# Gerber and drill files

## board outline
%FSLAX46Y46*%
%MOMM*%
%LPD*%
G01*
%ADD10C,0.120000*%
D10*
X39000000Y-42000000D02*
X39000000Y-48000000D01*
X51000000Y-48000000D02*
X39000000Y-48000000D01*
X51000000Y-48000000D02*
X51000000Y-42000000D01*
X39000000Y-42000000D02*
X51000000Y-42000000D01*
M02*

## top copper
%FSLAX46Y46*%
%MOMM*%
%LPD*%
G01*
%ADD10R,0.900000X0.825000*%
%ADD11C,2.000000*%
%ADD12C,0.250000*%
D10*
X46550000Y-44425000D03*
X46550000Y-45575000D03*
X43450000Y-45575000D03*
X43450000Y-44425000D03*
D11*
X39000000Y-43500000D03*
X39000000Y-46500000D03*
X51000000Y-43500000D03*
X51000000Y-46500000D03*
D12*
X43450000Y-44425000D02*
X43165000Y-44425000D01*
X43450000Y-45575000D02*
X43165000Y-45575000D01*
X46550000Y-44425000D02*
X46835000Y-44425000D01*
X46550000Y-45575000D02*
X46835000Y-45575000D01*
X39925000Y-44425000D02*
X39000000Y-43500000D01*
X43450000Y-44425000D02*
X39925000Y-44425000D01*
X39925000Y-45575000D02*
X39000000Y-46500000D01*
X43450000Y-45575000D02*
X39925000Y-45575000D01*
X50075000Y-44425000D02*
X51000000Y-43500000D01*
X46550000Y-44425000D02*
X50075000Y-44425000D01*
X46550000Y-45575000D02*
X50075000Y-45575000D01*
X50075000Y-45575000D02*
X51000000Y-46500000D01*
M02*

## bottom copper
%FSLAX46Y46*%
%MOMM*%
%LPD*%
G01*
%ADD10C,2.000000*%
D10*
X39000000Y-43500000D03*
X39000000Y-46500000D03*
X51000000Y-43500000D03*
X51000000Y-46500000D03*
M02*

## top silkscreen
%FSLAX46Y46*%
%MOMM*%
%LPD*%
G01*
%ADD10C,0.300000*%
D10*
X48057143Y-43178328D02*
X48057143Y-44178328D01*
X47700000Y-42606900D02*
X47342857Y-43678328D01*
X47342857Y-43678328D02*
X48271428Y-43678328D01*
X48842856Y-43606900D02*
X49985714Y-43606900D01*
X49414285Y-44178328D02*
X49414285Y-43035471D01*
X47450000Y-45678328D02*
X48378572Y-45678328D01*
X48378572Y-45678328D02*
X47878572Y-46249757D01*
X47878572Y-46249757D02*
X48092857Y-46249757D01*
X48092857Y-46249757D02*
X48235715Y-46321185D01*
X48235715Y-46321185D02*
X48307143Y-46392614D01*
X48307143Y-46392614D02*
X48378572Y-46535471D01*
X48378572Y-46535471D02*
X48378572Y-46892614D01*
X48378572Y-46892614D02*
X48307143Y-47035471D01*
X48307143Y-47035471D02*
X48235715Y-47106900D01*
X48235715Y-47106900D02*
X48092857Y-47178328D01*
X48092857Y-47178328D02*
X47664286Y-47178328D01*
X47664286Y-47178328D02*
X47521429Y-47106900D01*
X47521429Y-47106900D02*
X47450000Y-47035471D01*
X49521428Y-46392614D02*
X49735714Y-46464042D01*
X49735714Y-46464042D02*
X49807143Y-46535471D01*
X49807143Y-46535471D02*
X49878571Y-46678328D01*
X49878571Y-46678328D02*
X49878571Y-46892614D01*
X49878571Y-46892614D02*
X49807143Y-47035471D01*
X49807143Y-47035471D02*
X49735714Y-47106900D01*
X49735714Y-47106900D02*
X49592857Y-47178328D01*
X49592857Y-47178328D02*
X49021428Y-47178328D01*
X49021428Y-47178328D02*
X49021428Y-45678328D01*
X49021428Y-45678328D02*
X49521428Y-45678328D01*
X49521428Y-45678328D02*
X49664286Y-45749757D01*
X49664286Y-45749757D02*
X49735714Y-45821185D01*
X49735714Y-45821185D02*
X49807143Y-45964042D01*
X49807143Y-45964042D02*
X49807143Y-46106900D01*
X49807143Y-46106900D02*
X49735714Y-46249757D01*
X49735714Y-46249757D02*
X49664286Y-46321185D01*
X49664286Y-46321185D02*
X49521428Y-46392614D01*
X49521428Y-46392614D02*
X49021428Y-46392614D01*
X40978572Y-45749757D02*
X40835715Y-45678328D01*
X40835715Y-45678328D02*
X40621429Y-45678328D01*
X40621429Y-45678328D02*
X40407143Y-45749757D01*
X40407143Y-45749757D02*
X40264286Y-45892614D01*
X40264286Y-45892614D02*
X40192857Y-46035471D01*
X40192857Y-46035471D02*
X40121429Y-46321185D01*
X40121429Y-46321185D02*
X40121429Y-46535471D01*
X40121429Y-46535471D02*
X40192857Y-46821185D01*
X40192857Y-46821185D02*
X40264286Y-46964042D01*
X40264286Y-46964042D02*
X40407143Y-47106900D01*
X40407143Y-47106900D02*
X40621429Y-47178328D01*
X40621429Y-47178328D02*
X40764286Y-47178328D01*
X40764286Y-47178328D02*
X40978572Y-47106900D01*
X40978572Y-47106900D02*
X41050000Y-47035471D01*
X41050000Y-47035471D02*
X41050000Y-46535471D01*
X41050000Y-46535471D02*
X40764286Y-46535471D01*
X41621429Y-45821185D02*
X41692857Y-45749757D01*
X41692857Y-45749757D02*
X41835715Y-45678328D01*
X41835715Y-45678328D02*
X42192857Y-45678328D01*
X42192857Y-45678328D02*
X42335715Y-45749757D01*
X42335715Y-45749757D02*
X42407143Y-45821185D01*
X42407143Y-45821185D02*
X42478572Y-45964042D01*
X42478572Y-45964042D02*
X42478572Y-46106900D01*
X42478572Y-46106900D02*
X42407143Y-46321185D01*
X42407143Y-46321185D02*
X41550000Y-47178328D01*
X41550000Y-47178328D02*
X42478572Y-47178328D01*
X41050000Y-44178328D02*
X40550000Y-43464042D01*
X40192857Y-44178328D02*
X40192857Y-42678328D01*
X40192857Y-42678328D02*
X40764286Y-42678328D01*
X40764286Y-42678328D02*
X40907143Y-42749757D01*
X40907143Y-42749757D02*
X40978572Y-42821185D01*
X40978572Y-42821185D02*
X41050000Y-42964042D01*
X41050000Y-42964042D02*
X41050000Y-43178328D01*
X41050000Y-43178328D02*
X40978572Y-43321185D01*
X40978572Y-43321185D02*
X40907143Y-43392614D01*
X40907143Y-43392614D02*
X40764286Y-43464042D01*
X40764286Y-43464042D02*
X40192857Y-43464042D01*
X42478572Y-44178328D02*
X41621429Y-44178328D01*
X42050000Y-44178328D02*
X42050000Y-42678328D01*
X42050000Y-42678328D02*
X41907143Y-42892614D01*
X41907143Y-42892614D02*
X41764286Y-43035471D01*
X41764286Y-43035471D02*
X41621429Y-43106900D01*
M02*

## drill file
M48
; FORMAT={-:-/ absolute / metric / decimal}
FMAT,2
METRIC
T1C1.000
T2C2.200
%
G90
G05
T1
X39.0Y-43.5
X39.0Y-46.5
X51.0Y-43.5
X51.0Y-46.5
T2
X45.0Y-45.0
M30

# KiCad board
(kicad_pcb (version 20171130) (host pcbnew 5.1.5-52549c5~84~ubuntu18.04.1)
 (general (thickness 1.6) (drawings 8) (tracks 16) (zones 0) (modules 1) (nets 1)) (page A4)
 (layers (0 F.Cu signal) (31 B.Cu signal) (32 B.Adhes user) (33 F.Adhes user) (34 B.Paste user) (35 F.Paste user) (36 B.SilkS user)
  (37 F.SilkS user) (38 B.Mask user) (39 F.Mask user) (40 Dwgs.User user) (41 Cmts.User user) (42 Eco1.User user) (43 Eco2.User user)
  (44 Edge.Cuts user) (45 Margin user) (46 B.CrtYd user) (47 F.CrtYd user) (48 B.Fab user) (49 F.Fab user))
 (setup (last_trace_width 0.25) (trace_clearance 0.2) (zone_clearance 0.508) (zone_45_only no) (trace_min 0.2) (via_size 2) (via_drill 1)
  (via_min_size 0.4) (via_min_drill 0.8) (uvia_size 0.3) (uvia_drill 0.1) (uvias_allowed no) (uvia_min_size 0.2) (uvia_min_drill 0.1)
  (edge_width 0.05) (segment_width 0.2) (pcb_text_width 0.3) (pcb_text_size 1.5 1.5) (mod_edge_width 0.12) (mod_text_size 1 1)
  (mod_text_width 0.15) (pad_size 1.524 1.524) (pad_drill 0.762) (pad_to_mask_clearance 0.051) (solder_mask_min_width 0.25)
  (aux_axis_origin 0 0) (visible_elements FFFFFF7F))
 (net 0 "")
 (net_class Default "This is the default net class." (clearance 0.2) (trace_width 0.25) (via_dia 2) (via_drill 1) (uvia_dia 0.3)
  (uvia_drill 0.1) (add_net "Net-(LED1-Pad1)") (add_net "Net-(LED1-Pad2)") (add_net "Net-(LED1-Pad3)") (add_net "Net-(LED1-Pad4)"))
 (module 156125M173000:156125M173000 (layer F.Cu) (at 45 45)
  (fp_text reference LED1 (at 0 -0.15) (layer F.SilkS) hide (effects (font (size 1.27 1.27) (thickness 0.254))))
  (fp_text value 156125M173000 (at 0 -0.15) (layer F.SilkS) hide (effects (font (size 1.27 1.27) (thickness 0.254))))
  (pad "" np_thru_hole circle (at 0 0 90) (size 2.2 2.2) (drill 2.2) (layers *.Cu *.Mask))
  (pad 4 smd rect (at 1.55 -0.575 90) (size 0.825 0.9) (layers F.Cu F.Paste F.Mask))
  (pad 3 smd rect (at 1.55 0.575 90) (size 0.825 0.9) (layers F.Cu F.Paste F.Mask))
  (pad 2 smd rect (at -1.55 0.575 90) (size 0.825 0.9) (layers F.Cu F.Paste F.Mask))
  (pad 1 smd rect (at -1.55 -0.575 90) (size 0.825 0.9) (layers F.Cu F.Paste F.Mask)))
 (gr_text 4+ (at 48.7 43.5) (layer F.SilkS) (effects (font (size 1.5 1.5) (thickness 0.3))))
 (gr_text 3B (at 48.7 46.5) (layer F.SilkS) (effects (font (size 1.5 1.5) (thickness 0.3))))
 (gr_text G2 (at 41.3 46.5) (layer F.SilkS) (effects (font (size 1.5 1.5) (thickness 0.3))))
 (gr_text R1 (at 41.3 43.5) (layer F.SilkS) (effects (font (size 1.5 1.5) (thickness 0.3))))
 (gr_line (start 39 42) (end 39 48) (layer Edge.Cuts) (width 0.12))
 (gr_line (start 51 48) (end 39 48) (layer Edge.Cuts) (width 0.12))
 (gr_line (start 51 48) (end 51 42) (layer Edge.Cuts) (width 0.12))
 (gr_line (start 39 42) (end 51 42) (layer Edge.Cuts) (width 0.12))
 (segment (start 43.45 44.425) (end 43.165 44.425) (width 0.25) (layer F.Cu) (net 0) (status 30))
 (segment (start 43.45 45.575) (end 43.165 45.575) (width 0.25) (layer F.Cu) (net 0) (status 30))
 (segment (start 46.55 44.425) (end 46.835 44.425) (width 0.25) (layer F.Cu) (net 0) (status 30))
 (segment (start 46.55 45.575) (end 46.835 45.575) (width 0.25) (layer F.Cu) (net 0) (status 30))
 (via (at 39 43.5) (size 2) (drill 1) (layers F.Cu B.Cu) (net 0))
 (via (at 39 46.5) (size 2) (drill 1) (layers F.Cu B.Cu) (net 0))
 (segment (start 39.925 44.425) (end 39 43.5) (width 0.25) (layer F.Cu) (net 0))
 (segment (start 43.45 44.425) (end 39.925 44.425) (width 0.25) (layer F.Cu) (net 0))
 (segment (start 39.925 45.575) (end 39 46.5) (width 0.25) (layer F.Cu) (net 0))
 (segment (start 43.45 45.575) (end 39.925 45.575) (width 0.25) (layer F.Cu) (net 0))
 (via (at 51 43.5) (size 2) (drill 1) (layers F.Cu B.Cu) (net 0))
 (segment (start 50.075 44.425) (end 51 43.5) (width 0.25) (layer F.Cu) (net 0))
 (segment (start 46.55 44.425) (end 50.075 44.425) (width 0.25) (layer F.Cu) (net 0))
 (via (at 51 46.5) (size 2) (drill 1) (layers F.Cu B.Cu) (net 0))
 (segment (start 46.55 45.575) (end 50.075 45.575) (width 0.25) (layer F.Cu) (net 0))
 (segment (start 50.075 45.575) (end 51 46.5) (width 0.25) (layer F.Cu) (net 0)))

